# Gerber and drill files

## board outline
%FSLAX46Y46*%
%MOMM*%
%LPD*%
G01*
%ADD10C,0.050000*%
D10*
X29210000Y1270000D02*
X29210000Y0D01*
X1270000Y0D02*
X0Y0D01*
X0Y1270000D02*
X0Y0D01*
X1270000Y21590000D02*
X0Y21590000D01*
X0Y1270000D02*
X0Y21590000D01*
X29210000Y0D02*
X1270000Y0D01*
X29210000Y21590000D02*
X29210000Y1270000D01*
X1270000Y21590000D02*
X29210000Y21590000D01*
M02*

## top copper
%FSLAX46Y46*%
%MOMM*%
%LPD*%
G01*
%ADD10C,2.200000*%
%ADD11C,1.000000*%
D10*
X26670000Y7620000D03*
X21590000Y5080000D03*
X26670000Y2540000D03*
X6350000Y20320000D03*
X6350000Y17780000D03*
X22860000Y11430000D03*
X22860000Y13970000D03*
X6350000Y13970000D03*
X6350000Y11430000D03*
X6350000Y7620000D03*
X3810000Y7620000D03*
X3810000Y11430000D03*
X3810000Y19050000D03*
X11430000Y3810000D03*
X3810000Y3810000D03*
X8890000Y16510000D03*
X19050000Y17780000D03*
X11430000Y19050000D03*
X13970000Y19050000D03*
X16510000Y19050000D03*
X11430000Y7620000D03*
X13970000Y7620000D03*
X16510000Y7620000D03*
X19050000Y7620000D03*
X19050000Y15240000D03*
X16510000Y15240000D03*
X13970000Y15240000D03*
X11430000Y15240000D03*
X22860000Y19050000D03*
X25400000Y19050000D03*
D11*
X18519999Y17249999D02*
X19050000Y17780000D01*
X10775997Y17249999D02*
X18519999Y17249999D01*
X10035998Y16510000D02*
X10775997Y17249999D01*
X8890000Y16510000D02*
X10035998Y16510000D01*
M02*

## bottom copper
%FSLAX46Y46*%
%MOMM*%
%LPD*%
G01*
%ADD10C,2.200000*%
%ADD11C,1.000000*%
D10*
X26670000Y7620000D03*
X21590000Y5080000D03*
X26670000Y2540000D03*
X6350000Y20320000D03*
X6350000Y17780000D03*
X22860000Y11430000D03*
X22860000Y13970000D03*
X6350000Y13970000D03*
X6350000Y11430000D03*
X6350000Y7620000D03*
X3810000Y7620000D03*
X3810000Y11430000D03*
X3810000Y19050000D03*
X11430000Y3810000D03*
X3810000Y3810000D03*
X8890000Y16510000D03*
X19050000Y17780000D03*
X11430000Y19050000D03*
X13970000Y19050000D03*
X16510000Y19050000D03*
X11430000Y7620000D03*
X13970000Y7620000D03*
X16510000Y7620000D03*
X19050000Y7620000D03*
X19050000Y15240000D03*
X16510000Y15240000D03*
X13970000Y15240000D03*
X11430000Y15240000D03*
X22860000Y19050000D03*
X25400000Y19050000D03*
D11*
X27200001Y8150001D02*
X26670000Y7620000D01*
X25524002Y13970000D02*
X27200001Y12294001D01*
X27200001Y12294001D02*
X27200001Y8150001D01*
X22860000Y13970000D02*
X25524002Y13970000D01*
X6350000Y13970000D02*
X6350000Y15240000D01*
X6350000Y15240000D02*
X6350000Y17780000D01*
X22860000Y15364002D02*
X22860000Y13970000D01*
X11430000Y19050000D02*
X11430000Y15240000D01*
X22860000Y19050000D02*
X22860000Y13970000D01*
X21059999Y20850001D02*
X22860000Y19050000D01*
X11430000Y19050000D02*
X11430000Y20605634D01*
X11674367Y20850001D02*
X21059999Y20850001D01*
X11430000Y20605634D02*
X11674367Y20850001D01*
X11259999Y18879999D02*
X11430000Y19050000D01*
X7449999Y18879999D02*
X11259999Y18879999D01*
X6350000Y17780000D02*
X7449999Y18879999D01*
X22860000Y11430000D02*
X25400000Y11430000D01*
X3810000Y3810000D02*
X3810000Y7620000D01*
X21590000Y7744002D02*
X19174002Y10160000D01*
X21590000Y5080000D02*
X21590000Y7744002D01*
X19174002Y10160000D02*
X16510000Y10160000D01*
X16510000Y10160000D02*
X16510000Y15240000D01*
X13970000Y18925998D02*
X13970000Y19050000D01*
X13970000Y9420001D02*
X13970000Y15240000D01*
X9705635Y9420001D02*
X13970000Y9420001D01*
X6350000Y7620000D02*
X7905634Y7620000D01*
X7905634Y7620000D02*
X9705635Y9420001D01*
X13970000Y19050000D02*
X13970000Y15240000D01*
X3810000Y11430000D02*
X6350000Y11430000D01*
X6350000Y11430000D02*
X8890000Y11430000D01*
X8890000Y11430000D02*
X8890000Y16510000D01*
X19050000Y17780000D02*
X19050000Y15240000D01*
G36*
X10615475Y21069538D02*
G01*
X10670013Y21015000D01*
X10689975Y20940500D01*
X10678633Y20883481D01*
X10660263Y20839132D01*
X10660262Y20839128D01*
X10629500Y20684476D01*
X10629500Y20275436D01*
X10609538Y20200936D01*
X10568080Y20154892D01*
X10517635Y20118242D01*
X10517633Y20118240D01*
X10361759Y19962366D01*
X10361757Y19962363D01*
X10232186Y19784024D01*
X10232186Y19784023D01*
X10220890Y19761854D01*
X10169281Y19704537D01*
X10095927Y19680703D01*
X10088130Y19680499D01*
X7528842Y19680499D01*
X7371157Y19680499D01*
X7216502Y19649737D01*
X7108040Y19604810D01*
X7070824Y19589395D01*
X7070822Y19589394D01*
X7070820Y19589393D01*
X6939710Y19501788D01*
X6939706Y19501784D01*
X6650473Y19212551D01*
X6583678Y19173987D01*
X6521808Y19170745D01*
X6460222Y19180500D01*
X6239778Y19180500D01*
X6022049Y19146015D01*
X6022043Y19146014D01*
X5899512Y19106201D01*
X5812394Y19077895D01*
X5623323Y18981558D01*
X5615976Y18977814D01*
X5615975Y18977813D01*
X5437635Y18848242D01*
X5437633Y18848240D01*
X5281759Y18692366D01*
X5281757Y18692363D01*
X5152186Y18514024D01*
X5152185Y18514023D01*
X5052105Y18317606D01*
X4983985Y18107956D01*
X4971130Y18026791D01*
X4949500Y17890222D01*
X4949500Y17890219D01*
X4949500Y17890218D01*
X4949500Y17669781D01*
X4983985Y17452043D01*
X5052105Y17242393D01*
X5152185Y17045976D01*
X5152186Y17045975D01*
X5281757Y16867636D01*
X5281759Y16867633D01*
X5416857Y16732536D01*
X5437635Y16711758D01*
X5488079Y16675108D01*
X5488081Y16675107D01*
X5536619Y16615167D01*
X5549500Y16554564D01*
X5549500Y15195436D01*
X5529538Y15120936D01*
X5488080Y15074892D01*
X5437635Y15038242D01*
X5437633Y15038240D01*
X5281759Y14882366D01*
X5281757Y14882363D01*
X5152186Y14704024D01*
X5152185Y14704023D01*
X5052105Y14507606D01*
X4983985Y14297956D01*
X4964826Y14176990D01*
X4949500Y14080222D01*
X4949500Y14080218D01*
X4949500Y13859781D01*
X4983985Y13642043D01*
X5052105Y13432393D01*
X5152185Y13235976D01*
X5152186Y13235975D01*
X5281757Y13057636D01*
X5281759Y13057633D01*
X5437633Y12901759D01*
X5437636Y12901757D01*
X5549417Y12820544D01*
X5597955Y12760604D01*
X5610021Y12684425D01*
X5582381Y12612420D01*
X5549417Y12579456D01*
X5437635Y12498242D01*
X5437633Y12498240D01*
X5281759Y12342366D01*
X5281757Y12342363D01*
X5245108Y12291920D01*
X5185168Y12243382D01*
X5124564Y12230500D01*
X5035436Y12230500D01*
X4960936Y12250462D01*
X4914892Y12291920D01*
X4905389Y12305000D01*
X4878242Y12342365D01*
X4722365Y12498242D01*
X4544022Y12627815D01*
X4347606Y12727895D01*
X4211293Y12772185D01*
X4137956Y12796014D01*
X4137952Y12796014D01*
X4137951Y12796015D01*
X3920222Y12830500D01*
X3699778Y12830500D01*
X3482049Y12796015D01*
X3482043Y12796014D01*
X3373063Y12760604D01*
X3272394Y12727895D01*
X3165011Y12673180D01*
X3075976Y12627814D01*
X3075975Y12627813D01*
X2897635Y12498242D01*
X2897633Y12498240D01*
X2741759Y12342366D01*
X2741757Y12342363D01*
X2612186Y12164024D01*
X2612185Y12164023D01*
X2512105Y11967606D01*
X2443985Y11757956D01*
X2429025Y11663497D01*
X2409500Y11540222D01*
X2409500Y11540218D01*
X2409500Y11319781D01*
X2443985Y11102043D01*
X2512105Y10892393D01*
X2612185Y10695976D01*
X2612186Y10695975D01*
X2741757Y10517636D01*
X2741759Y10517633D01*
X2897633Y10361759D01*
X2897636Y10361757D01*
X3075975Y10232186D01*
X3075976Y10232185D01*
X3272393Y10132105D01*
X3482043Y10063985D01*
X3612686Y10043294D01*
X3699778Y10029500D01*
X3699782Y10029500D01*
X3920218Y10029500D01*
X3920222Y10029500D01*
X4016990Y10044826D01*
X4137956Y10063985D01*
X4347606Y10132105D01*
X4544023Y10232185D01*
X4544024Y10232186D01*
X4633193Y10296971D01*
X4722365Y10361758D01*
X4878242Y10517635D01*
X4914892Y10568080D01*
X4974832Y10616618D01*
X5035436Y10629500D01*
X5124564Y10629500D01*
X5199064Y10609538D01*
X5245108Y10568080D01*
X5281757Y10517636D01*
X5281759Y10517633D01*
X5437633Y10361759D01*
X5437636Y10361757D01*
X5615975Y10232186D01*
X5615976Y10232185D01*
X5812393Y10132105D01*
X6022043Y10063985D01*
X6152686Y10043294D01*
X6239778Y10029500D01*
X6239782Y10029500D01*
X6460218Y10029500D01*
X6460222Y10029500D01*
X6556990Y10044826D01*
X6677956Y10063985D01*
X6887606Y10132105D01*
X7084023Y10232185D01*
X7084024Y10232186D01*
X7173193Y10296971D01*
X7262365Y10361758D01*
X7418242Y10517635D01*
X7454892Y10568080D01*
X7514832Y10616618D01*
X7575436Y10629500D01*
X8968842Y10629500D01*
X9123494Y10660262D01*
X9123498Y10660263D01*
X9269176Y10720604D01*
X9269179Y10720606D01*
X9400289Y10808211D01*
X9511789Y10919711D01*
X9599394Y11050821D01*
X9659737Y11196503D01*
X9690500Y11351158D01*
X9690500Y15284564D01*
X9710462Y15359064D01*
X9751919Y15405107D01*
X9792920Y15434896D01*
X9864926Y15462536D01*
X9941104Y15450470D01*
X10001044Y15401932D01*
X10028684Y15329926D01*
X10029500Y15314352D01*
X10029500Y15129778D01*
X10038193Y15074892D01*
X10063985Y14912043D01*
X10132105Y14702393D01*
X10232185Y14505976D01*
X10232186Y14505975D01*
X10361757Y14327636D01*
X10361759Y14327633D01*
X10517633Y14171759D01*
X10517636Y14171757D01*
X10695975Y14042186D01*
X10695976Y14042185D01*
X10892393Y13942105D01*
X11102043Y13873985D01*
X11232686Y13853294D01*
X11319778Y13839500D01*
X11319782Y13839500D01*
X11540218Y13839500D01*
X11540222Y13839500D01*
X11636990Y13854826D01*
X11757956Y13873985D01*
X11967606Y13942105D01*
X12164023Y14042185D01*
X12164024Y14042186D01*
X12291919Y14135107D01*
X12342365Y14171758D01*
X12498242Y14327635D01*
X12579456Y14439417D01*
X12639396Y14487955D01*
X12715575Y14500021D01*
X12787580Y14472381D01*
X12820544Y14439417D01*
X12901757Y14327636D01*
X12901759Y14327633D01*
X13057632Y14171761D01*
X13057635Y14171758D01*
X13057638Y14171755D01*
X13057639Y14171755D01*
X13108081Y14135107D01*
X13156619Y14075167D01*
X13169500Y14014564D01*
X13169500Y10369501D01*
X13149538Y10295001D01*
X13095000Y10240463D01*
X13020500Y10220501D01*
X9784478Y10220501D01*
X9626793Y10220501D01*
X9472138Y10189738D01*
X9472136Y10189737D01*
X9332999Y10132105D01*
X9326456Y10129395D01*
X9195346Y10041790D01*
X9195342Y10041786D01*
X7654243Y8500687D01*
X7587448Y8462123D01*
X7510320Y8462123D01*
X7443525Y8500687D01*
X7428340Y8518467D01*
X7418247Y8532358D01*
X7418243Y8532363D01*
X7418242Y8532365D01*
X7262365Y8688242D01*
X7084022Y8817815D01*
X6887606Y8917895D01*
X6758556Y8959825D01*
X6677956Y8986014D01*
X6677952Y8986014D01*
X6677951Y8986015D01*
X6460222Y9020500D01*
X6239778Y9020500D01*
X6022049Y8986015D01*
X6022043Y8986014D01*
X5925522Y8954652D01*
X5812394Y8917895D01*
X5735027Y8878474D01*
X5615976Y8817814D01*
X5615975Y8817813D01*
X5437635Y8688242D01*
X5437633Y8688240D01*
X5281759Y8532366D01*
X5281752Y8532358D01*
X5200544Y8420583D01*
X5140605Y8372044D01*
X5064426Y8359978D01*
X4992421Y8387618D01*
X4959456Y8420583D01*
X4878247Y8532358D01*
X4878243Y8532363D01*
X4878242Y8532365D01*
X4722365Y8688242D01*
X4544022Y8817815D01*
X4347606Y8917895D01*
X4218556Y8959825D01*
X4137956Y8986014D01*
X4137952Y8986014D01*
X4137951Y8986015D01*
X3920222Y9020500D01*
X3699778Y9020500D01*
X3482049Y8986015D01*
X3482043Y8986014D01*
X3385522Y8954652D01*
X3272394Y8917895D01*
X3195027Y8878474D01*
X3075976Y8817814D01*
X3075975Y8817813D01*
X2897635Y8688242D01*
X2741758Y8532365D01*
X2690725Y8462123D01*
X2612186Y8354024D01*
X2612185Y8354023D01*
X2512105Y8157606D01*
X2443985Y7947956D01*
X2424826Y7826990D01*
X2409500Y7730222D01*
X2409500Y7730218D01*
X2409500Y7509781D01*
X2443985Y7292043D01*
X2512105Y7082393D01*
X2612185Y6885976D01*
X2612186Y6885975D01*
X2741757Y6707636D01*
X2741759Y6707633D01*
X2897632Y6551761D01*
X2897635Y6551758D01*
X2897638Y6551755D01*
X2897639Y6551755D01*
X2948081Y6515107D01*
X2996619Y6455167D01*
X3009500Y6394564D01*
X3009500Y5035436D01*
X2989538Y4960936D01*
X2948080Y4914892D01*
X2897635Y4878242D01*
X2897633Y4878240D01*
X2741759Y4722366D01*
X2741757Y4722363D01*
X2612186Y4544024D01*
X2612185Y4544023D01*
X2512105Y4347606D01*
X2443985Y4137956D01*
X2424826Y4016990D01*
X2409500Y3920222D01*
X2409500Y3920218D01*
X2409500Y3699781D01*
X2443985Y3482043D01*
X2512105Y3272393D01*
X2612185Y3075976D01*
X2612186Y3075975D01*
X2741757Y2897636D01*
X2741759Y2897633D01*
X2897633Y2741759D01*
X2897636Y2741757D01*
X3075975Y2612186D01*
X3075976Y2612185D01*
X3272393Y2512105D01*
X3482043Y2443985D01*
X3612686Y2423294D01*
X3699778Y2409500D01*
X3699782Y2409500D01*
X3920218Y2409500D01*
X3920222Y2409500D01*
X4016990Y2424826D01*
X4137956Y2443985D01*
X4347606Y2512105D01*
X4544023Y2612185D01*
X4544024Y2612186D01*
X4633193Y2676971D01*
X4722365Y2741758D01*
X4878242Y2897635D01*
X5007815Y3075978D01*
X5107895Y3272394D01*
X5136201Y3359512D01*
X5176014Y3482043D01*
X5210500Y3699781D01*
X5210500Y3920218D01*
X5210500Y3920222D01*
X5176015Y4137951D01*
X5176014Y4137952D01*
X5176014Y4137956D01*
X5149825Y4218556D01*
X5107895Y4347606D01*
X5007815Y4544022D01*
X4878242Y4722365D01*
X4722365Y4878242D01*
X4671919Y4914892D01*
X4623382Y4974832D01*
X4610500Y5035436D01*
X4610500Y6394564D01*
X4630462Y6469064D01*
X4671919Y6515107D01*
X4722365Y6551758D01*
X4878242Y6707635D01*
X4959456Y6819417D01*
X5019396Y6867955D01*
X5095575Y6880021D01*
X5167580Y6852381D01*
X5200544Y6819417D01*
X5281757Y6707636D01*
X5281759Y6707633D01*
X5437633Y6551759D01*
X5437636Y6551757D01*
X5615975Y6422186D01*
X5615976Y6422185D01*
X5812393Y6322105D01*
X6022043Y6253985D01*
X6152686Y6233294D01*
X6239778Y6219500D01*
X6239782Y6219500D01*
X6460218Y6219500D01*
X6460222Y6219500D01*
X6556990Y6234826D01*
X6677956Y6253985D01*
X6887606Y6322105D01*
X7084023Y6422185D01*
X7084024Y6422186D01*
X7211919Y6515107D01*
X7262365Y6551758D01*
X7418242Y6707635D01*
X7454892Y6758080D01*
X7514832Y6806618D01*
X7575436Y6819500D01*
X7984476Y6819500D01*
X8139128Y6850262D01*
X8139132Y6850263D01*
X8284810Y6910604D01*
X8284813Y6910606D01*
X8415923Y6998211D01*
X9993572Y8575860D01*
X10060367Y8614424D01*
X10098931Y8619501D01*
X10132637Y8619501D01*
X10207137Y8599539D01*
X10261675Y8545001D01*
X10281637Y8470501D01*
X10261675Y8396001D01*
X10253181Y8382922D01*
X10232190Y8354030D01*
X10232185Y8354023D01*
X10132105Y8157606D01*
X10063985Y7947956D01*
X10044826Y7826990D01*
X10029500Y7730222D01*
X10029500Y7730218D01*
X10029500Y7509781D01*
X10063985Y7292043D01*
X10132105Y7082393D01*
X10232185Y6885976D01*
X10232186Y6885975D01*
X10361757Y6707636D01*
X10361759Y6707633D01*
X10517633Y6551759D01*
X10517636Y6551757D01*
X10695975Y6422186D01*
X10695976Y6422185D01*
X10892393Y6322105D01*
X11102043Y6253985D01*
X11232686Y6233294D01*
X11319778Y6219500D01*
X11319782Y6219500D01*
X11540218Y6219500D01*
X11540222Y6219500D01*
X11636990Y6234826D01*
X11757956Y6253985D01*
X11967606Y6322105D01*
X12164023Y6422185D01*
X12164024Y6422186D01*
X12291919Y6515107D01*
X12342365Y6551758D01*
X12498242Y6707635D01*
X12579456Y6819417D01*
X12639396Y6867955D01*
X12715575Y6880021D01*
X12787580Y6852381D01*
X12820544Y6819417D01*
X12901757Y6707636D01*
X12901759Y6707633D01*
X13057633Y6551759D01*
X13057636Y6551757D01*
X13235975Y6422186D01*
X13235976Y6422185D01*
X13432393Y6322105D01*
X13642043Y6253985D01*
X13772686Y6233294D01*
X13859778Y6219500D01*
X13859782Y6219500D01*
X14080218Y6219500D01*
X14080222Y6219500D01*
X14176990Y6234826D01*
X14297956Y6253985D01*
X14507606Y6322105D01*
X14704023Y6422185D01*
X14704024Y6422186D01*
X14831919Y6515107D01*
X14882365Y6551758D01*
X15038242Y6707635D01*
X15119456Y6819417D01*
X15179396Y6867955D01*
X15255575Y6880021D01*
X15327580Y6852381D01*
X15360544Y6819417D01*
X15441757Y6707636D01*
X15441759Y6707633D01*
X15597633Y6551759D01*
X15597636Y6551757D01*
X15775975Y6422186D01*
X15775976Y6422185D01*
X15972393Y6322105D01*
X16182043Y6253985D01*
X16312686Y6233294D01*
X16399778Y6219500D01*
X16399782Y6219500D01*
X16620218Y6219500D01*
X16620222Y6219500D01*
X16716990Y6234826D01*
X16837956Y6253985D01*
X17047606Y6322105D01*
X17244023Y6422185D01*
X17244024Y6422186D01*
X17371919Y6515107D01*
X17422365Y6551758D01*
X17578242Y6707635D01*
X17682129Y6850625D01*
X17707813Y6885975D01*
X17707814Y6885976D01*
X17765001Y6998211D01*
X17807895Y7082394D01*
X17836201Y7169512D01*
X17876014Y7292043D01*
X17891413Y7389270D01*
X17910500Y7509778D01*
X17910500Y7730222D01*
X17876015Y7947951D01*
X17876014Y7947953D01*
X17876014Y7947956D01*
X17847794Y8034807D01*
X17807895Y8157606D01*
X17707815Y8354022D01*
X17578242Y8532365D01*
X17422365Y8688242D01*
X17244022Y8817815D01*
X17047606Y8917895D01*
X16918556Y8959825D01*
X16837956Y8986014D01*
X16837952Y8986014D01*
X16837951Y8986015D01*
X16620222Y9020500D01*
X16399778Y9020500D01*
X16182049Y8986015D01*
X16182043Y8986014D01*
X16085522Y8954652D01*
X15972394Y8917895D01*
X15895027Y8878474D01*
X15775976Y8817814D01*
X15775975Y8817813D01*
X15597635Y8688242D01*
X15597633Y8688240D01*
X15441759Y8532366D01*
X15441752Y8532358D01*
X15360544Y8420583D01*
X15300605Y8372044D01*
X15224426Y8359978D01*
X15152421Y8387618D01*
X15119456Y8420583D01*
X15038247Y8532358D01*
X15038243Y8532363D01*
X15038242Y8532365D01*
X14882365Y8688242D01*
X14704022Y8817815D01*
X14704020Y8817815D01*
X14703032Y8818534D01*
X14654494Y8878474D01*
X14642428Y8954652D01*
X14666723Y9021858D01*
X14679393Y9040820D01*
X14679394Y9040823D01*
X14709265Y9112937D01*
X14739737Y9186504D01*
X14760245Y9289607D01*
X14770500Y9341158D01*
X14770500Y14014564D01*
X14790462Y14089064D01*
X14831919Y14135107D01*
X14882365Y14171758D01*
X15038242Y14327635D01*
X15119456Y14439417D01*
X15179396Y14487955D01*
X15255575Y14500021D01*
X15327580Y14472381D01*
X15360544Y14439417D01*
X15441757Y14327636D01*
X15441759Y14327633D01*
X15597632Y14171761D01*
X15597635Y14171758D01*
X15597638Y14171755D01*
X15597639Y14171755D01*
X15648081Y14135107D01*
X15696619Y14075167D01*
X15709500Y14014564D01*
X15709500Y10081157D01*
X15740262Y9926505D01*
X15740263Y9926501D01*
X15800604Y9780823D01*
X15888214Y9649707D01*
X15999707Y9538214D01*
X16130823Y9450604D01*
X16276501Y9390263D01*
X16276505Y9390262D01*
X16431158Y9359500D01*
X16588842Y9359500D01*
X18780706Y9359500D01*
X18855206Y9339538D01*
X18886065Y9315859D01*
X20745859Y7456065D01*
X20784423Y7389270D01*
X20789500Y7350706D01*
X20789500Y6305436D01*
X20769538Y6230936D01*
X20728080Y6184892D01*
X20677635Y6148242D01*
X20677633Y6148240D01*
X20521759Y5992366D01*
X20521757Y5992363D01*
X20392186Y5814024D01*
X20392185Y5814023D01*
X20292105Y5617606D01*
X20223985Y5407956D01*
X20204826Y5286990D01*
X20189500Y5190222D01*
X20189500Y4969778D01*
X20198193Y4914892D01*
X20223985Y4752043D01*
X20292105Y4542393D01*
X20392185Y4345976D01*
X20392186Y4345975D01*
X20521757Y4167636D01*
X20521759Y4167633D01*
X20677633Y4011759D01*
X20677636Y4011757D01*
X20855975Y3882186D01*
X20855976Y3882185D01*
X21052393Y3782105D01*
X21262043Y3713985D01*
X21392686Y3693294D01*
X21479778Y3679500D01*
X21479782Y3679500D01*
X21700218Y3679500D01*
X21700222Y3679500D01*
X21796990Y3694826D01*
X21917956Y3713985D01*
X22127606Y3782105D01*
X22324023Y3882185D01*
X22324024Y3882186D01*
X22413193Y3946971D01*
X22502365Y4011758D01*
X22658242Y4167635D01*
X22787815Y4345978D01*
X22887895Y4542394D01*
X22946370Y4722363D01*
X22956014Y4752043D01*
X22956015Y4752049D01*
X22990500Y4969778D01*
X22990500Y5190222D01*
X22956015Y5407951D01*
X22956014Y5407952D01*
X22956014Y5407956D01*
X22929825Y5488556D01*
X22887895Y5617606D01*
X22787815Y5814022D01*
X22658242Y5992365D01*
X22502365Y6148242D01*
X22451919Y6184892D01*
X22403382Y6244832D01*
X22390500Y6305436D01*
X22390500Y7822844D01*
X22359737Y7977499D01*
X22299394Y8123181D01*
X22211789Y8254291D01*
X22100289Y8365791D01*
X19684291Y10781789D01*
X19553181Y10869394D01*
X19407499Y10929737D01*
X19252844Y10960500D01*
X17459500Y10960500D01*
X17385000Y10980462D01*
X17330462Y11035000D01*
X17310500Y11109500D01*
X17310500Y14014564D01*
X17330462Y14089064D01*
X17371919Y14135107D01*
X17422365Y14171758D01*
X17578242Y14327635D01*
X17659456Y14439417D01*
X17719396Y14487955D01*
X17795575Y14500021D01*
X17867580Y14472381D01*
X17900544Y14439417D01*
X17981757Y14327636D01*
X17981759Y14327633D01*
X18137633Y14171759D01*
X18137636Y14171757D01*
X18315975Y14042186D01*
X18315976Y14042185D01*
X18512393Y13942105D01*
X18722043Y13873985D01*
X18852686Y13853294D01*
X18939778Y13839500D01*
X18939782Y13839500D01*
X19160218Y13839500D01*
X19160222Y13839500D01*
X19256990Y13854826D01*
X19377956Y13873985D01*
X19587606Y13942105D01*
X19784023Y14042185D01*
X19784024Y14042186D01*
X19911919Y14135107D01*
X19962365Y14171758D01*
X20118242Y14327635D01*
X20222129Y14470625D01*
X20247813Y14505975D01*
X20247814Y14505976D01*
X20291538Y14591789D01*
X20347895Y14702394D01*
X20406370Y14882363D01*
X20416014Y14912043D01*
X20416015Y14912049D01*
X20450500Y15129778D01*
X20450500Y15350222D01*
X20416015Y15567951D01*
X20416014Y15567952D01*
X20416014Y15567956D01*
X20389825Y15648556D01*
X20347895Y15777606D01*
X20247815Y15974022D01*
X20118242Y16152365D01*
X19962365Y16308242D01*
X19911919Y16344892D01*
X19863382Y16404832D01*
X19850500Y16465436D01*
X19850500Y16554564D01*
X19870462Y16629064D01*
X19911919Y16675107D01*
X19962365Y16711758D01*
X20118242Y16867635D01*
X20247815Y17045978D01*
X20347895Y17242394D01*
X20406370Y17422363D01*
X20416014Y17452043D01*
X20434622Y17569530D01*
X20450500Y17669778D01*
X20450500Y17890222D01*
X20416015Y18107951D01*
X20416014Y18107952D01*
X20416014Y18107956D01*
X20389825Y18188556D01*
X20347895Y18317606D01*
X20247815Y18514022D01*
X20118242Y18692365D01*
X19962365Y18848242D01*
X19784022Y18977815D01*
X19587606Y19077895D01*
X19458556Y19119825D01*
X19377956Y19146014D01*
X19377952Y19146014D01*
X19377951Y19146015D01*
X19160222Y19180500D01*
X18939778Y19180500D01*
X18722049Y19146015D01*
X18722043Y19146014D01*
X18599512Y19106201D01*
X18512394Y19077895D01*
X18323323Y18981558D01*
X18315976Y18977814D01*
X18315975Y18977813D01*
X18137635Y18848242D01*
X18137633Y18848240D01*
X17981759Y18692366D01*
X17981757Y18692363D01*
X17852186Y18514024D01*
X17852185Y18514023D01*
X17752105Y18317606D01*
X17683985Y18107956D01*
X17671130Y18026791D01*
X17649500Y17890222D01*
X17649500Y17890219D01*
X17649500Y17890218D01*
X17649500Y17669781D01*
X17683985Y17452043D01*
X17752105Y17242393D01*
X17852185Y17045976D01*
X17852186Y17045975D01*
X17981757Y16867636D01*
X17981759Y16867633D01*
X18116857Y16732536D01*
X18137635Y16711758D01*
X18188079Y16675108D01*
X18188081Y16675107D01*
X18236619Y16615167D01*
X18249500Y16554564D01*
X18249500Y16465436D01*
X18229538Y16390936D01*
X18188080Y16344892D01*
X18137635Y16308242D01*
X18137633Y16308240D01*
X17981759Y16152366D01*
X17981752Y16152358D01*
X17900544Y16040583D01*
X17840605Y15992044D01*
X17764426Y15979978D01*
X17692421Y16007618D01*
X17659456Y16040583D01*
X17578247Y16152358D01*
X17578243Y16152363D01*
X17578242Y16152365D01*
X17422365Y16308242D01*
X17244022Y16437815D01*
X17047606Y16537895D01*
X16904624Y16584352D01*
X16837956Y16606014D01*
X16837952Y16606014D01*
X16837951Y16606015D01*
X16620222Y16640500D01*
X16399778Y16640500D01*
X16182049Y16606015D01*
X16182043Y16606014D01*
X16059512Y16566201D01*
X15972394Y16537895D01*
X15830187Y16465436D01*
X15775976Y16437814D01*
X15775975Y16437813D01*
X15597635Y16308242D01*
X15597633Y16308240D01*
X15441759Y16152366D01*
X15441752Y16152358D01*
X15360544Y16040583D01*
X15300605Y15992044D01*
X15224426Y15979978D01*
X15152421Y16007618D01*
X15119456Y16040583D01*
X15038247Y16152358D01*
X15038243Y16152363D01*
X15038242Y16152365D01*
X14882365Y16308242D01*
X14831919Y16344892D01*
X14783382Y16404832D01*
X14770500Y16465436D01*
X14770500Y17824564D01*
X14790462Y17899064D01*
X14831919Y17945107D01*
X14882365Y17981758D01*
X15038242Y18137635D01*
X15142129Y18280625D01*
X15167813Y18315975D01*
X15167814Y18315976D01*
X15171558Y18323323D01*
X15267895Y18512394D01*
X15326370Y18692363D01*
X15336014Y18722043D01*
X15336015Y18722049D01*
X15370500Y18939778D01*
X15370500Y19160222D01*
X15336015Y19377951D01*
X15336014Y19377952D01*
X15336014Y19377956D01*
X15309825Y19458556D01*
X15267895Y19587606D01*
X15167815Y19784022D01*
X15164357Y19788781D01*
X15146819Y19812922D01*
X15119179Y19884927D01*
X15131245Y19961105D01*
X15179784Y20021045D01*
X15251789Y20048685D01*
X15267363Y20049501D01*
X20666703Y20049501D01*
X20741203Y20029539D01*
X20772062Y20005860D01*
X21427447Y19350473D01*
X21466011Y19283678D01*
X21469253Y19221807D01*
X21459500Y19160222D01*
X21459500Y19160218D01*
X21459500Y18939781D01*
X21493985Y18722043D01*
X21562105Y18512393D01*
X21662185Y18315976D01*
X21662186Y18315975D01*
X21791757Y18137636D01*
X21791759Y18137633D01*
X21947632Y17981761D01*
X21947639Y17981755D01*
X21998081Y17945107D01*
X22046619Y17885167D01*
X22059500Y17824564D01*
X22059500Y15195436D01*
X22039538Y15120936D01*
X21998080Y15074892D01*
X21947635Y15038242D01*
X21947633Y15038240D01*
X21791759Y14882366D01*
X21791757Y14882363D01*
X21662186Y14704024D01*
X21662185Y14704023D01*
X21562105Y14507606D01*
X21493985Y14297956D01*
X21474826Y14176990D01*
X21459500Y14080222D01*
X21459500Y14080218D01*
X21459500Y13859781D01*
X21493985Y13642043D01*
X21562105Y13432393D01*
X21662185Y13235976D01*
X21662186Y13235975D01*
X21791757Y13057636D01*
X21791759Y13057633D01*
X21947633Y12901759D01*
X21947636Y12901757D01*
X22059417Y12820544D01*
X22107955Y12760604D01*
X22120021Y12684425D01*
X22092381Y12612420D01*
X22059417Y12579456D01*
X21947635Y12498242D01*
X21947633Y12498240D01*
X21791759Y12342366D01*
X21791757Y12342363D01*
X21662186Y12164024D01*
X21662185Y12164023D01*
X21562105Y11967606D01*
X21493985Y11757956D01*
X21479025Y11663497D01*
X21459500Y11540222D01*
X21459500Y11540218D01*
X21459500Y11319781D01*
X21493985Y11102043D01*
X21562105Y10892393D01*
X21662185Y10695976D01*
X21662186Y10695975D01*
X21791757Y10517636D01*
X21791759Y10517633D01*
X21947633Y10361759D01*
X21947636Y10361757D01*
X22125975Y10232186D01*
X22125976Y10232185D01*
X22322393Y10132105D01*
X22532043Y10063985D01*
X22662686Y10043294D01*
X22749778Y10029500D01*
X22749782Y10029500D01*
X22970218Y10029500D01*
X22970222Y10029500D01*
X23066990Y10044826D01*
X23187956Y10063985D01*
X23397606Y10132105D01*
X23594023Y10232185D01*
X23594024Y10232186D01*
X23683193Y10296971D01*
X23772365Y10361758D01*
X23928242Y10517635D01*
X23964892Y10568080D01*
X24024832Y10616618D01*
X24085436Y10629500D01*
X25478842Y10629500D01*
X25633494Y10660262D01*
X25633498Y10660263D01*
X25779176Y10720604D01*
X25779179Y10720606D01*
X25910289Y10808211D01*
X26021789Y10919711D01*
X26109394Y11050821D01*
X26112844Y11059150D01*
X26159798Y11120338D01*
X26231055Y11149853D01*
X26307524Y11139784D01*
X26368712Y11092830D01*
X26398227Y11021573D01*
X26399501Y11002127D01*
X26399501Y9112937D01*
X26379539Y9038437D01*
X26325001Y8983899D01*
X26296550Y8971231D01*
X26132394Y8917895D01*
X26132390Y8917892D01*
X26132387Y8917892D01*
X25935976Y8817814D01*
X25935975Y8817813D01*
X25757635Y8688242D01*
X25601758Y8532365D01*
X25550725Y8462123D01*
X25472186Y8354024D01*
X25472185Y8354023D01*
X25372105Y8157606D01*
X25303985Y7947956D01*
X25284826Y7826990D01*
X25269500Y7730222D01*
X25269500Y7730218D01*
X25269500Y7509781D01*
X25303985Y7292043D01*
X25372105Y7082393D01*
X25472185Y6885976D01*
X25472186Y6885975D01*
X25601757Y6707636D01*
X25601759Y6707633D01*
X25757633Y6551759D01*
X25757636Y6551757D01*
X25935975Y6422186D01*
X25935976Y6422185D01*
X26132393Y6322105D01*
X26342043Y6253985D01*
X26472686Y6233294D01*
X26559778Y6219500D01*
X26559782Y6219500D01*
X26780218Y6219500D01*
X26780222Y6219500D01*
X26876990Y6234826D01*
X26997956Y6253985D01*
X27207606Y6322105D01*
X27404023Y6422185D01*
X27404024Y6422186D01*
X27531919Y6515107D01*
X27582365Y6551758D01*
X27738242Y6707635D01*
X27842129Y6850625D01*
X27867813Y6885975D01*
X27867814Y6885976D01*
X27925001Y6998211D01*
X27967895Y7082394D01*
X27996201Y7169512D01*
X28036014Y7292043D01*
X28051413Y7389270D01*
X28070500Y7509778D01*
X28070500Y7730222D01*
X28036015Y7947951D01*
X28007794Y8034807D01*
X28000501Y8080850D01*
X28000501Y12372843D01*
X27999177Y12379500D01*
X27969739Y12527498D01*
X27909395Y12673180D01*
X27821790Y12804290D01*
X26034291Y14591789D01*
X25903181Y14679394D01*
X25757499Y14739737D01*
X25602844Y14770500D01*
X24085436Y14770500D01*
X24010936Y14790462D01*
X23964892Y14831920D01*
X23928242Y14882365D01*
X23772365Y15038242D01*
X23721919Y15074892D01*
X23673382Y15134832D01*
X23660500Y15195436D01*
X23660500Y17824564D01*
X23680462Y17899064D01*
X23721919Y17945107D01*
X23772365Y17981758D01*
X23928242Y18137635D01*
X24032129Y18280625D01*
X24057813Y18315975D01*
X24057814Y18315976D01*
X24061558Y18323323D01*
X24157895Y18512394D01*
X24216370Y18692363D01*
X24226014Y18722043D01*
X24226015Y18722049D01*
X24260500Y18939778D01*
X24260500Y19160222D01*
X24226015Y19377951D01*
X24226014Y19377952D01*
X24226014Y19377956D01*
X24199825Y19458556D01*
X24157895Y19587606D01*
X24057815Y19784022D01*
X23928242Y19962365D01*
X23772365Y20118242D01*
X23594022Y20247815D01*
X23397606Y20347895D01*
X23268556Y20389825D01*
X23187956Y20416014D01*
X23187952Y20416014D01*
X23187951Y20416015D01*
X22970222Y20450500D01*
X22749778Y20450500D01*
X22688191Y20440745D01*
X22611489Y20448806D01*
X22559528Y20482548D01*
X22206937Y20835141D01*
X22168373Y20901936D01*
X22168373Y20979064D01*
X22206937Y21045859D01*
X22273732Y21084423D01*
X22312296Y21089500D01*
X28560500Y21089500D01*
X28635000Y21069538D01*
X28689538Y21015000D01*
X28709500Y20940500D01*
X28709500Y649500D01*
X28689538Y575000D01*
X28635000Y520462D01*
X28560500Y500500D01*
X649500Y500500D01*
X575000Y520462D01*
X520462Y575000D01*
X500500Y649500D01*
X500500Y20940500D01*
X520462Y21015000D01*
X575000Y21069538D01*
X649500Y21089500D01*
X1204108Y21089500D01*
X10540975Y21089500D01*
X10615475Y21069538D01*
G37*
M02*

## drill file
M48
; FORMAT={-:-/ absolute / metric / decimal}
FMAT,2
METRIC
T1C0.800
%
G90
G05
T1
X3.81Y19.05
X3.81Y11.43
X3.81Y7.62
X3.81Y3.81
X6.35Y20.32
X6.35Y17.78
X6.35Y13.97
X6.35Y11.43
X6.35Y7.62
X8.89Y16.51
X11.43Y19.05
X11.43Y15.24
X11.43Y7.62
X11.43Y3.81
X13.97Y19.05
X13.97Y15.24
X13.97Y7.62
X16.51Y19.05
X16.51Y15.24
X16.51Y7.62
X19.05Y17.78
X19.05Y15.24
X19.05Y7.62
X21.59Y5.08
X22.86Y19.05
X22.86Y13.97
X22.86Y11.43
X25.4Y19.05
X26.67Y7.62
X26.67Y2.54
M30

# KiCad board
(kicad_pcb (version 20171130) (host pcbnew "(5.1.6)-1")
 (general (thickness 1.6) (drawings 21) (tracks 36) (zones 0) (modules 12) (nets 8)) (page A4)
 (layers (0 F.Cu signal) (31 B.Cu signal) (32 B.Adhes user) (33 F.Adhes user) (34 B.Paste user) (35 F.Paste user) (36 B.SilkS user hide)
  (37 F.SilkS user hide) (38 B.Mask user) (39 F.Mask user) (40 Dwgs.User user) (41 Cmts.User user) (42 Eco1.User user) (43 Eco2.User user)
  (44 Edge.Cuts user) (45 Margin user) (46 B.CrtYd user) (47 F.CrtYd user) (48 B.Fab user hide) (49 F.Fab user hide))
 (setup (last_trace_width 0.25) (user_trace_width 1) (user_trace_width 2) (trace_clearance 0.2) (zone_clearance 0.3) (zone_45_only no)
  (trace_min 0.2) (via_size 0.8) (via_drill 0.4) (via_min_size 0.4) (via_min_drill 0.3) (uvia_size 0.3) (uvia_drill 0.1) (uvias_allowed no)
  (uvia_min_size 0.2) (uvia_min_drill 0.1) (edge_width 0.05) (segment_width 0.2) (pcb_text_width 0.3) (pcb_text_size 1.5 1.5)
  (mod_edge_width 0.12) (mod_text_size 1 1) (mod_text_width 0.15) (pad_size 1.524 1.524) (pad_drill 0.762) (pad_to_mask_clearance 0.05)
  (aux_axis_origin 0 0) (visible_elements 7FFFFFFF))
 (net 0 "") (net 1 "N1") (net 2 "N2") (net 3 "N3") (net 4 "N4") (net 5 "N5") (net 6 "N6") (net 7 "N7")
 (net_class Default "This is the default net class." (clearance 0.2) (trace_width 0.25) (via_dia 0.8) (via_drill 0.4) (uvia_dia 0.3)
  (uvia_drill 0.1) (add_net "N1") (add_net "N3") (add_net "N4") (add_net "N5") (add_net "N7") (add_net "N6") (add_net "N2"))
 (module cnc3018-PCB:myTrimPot (layer F.Cu) (at 24.13 -5.08 270)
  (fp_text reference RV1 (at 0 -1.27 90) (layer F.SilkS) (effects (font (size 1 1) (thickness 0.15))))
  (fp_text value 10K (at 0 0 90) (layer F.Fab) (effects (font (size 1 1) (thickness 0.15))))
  (pad 1 thru_hole circle (at -2.54 -2.54 270) (size 2.2 2.2) (drill 0.8) (layers *.Cu *.Mask) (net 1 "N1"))
  (pad 2 thru_hole circle (at 0 2.54 270) (size 2.2 2.2) (drill 0.8) (layers *.Cu *.Mask) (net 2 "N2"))
  (pad 3 thru_hole circle (at 2.54 -2.54 270) (size 2.2 2.2) (drill 0.8) (layers *.Cu *.Mask) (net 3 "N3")))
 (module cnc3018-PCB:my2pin (layer F.Cu) (at 6.35 -17.78 90)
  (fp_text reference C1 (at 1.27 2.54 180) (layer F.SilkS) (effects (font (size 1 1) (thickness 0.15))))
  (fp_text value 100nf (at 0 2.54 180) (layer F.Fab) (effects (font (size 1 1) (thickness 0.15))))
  (pad 2 thru_hole circle (at 2.54 0 90) (size 2.2 2.2) (drill 0.8) (layers *.Cu *.Mask) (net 3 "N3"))
  (pad 1 thru_hole circle (at 0 0 90) (size 2.2 2.2) (drill 0.8) (layers *.Cu *.Mask) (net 1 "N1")))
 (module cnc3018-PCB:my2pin (layer F.Cu) (at 22.86 -11.43 90)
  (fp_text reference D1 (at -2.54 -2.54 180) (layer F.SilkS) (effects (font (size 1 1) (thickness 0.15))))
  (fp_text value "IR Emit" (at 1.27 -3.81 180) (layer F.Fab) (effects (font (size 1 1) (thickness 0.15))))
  (pad 1 thru_hole circle (at 0 0 90) (size 2.2 2.2) (drill 0.8) (layers *.Cu *.Mask) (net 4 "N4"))
  (pad 2 thru_hole circle (at 2.54 0 90) (size 2.2 2.2) (drill 0.8) (layers *.Cu *.Mask) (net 1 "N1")))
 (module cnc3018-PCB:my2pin (layer F.Cu) (at 6.35 -13.97 270)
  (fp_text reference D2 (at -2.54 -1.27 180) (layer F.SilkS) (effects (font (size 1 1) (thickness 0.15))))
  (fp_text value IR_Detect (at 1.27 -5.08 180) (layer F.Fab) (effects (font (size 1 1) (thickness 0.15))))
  (pad 1 thru_hole circle (at 0 0 270) (size 2.2 2.2) (drill 0.8) (layers *.Cu *.Mask) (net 1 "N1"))
  (pad 2 thru_hole circle (at 2.54 0 270) (size 2.2 2.2) (drill 0.8) (layers *.Cu *.Mask) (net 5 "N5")))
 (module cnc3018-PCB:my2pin (layer F.Cu) (at 3.81 -7.62)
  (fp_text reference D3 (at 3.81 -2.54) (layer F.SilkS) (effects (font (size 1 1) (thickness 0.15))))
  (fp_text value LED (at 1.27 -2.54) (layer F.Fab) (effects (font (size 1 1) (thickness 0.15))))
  (pad 2 thru_hole circle (at 2.54 0) (size 2.2 2.2) (drill 0.8) (layers *.Cu *.Mask) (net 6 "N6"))
  (pad 1 thru_hole circle (at 0 0) (size 2.2 2.2) (drill 0.8) (layers *.Cu *.Mask) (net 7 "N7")))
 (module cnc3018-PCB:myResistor (layer F.Cu) (at 3.81 -19.05 270)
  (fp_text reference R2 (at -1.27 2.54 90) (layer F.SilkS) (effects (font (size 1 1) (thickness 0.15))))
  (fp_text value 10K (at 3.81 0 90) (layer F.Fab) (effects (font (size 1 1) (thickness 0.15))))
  (pad 2 thru_hole circle (at 7.62 0 270) (size 2.2 2.2) (drill 0.8) (layers *.Cu *.Mask) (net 5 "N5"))
  (pad 1 thru_hole circle (at 0 0 270) (size 2.2 2.2) (drill 0.8) (layers *.Cu *.Mask) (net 3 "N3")))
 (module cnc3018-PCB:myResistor (layer F.Cu) (at 11.43 -3.81 180)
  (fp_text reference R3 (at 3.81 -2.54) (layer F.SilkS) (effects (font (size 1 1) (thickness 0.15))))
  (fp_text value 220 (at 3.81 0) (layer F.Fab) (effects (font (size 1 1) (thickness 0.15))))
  (pad 1 thru_hole circle (at 0 0 180) (size 2.2 2.2) (drill 0.8) (layers *.Cu *.Mask) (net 3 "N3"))
  (pad 2 thru_hole circle (at 7.62 0 180) (size 2.2 2.2) (drill 0.8) (layers *.Cu *.Mask) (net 7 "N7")))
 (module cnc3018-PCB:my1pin (layer F.Cu) (at 8.89 -16.51)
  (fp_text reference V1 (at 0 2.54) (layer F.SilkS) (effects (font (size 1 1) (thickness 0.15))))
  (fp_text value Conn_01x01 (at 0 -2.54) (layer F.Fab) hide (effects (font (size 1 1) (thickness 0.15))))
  (pad 1 thru_hole circle (at 0 0) (size 2.2 2.2) (drill 0.8) (layers *.Cu *.Mask) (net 5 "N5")))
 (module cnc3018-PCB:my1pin (layer F.Cu) (at 19.05 -17.78)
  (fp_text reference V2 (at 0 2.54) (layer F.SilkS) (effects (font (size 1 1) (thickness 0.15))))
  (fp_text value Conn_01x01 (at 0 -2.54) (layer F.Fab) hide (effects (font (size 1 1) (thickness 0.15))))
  (pad 1 thru_hole circle (at 0 0) (size 2.2 2.2) (drill 0.8) (layers *.Cu *.Mask) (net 5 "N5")))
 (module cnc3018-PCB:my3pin (layer F.Cu) (at 13.97 -19.05)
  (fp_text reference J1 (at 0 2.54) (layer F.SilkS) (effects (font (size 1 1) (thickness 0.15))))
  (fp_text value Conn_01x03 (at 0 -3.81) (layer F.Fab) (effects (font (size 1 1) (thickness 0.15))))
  (pad 1 thru_hole circle (at -2.54 0) (size 2.2 2.2) (drill 0.8) (layers *.Cu *.Mask) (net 1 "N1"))
  (pad 2 thru_hole circle (at 0 0) (size 2.2 2.2) (drill 0.8) (layers *.Cu *.Mask) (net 6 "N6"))
  (pad 3 thru_hole circle (at 2.54 0) (size 2.2 2.2) (drill 0.8) (layers *.Cu *.Mask) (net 3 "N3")))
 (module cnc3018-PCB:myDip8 (layer F.Cu) (at 11.43 -7.62 90)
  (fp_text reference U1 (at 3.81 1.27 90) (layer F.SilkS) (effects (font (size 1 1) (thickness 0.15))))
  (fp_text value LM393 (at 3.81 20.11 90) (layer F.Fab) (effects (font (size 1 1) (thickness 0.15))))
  (pad 1 thru_hole circle (at 0 0 90) (size 2.2 2.2) (drill 0.8) (layers *.Cu *.Mask))
  (pad 2 thru_hole circle (at 0 2.54 90) (size 2.2 2.2) (drill 0.8) (layers *.Cu *.Mask))
  (pad 3 thru_hole circle (at 0 5.08 90) (size 2.2 2.2) (drill 0.8) (layers *.Cu *.Mask))
  (pad 4 thru_hole circle (at 0 7.62 90) (size 2.2 2.2) (drill 0.8) (layers *.Cu *.Mask) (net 3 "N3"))
  (pad 5 thru_hole circle (at 7.62 7.62 90) (size 2.2 2.2) (drill 0.8) (layers *.Cu *.Mask) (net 5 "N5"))
  (pad 6 thru_hole circle (at 7.62 5.08 90) (size 2.2 2.2) (drill 0.8) (layers *.Cu *.Mask) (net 2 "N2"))
  (pad 7 thru_hole circle (at 7.62 2.54 90) (size 2.2 2.2) (drill 0.8) (layers *.Cu *.Mask) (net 6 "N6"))
  (pad 8 thru_hole circle (at 7.62 0 90) (size 2.2 2.2) (drill 0.8) (layers *.Cu *.Mask) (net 1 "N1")))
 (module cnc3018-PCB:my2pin (layer F.Cu) (at 22.86 -19.05)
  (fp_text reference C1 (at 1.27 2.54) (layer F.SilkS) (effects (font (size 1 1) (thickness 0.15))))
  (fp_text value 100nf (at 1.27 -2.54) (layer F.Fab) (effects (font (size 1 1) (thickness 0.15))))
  (pad 1 thru_hole circle (at 0 0) (size 2.2 2.2) (drill 0.8) (layers *.Cu *.Mask) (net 1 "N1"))
  (pad 2 thru_hole circle (at 2.54 0) (size 2.2 2.2) (drill 0.8) (layers *.Cu *.Mask) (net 3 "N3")))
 (gr_line (start 29.21 -1.27) (end 29.21 0) (layer Edge.Cuts) (width 0.05))
 (gr_line (start 1.27 0) (end 0 0) (layer Edge.Cuts) (width 0.05))
 (gr_line (start 0 -1.27) (end 0 0) (layer Edge.Cuts) (width 0.05))
 (gr_line (start 1.27 -21.59) (end 0 -21.59) (layer Edge.Cuts) (width 0.05))
 (gr_line (start 0 -1.27) (end 0 -21.59) (layer Edge.Cuts) (width 0.05))
 (gr_line (start 29.21 0) (end 1.27 0) (layer Edge.Cuts) (width 0.05))
 (gr_line (start 29.21 -21.59) (end 29.21 -1.27) (layer Edge.Cuts) (width 0.05))
 (gr_line (start 1.27 -21.59) (end 29.21 -21.59) (layer Edge.Cuts) (width 0.05))
 (segment (start 27.200001 -8.150001) (end 26.67 -7.62) (width 1) (layer B.Cu) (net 1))
 (segment (start 25.524002 -13.97) (end 27.200001 -12.294001) (width 1) (layer B.Cu) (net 1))
 (segment (start 27.200001 -12.294001) (end 27.200001 -8.150001) (width 1) (layer B.Cu) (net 1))
 (segment (start 22.86 -13.97) (end 25.524002 -13.97) (width 1) (layer B.Cu) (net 1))
 (segment (start 6.35 -13.97) (end 6.35 -15.24) (width 1) (layer B.Cu) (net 1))
 (segment (start 6.35 -15.24) (end 6.35 -17.78) (width 1) (layer B.Cu) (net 1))
 (segment (start 22.86 -15.364002) (end 22.86 -13.97) (width 1) (layer B.Cu) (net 1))
 (segment (start 11.43 -19.05) (end 11.43 -15.24) (width 1) (layer B.Cu) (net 1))
 (segment (start 22.86 -19.05) (end 22.86 -13.97) (width 1) (layer B.Cu) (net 1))
 (segment (start 21.059999 -20.850001) (end 22.86 -19.05) (width 1) (layer B.Cu) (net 1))
 (segment (start 11.43 -19.05) (end 11.43 -20.605634) (width 1) (layer B.Cu) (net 1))
 (segment (start 11.674367 -20.850001) (end 21.059999 -20.850001) (width 1) (layer B.Cu) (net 1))
 (segment (start 11.43 -20.605634) (end 11.674367 -20.850001) (width 1) (layer B.Cu) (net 1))
 (segment (start 11.259999 -18.879999) (end 11.43 -19.05) (width 1) (layer B.Cu) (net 1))
 (segment (start 7.449999 -18.879999) (end 11.259999 -18.879999) (width 1) (layer B.Cu) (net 1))
 (segment (start 6.35 -17.78) (end 7.449999 -18.879999) (width 1) (layer B.Cu) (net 1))
 (segment (start 22.86 -11.43) (end 25.4 -11.43) (width 1) (layer B.Cu) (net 4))
 (segment (start 3.81 -3.81) (end 3.81 -7.62) (width 1) (layer B.Cu) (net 7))
 (segment (start 21.59 -7.744002) (end 19.174002 -10.16) (width 1) (layer B.Cu) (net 2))
 (segment (start 21.59 -5.08) (end 21.59 -7.744002) (width 1) (layer B.Cu) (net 2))
 (segment (start 19.174002 -10.16) (end 16.51 -10.16) (width 1) (layer B.Cu) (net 2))
 (segment (start 16.51 -10.16) (end 16.51 -15.24) (width 1) (layer B.Cu) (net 2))
 (segment (start 13.97 -18.925998) (end 13.97 -19.05) (width 1) (layer B.Cu) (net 6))
 (segment (start 13.97 -9.420001) (end 13.97 -15.24) (width 1) (layer B.Cu) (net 6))
 (segment (start 9.705635 -9.420001) (end 13.97 -9.420001) (width 1) (layer B.Cu) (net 6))
 (segment (start 6.35 -7.62) (end 7.905634 -7.62) (width 1) (layer B.Cu) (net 6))
 (segment (start 7.905634 -7.62) (end 9.705635 -9.420001) (width 1) (layer B.Cu) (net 6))
 (segment (start 13.97 -19.05) (end 13.97 -15.24) (width 1) (layer B.Cu) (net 6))
 (segment (start 3.81 -11.43) (end 6.35 -11.43) (width 1) (layer B.Cu) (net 5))
 (segment (start 6.35 -11.43) (end 8.89 -11.43) (width 1) (layer B.Cu) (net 5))
 (segment (start 8.89 -11.43) (end 8.89 -16.51) (width 1) (layer B.Cu) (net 5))
 (segment (start 19.05 -17.78) (end 19.05 -15.24) (width 1) (layer B.Cu) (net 5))
 (segment (start 18.519999 -17.249999) (end 19.05 -17.78) (width 1) (layer F.Cu) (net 5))
 (segment (start 10.775997 -17.249999) (end 18.519999 -17.249999) (width 1) (layer F.Cu) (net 5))
 (segment (start 10.035998 -16.51) (end 10.775997 -17.249999) (width 1) (layer F.Cu) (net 5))
 (segment (start 8.89 -16.51) (end 10.035998 -16.51) (width 1) (layer F.Cu) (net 5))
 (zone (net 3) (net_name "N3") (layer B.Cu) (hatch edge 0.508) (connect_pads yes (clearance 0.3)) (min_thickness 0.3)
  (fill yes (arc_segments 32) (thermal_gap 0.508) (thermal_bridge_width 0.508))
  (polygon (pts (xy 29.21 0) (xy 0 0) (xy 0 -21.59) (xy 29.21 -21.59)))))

